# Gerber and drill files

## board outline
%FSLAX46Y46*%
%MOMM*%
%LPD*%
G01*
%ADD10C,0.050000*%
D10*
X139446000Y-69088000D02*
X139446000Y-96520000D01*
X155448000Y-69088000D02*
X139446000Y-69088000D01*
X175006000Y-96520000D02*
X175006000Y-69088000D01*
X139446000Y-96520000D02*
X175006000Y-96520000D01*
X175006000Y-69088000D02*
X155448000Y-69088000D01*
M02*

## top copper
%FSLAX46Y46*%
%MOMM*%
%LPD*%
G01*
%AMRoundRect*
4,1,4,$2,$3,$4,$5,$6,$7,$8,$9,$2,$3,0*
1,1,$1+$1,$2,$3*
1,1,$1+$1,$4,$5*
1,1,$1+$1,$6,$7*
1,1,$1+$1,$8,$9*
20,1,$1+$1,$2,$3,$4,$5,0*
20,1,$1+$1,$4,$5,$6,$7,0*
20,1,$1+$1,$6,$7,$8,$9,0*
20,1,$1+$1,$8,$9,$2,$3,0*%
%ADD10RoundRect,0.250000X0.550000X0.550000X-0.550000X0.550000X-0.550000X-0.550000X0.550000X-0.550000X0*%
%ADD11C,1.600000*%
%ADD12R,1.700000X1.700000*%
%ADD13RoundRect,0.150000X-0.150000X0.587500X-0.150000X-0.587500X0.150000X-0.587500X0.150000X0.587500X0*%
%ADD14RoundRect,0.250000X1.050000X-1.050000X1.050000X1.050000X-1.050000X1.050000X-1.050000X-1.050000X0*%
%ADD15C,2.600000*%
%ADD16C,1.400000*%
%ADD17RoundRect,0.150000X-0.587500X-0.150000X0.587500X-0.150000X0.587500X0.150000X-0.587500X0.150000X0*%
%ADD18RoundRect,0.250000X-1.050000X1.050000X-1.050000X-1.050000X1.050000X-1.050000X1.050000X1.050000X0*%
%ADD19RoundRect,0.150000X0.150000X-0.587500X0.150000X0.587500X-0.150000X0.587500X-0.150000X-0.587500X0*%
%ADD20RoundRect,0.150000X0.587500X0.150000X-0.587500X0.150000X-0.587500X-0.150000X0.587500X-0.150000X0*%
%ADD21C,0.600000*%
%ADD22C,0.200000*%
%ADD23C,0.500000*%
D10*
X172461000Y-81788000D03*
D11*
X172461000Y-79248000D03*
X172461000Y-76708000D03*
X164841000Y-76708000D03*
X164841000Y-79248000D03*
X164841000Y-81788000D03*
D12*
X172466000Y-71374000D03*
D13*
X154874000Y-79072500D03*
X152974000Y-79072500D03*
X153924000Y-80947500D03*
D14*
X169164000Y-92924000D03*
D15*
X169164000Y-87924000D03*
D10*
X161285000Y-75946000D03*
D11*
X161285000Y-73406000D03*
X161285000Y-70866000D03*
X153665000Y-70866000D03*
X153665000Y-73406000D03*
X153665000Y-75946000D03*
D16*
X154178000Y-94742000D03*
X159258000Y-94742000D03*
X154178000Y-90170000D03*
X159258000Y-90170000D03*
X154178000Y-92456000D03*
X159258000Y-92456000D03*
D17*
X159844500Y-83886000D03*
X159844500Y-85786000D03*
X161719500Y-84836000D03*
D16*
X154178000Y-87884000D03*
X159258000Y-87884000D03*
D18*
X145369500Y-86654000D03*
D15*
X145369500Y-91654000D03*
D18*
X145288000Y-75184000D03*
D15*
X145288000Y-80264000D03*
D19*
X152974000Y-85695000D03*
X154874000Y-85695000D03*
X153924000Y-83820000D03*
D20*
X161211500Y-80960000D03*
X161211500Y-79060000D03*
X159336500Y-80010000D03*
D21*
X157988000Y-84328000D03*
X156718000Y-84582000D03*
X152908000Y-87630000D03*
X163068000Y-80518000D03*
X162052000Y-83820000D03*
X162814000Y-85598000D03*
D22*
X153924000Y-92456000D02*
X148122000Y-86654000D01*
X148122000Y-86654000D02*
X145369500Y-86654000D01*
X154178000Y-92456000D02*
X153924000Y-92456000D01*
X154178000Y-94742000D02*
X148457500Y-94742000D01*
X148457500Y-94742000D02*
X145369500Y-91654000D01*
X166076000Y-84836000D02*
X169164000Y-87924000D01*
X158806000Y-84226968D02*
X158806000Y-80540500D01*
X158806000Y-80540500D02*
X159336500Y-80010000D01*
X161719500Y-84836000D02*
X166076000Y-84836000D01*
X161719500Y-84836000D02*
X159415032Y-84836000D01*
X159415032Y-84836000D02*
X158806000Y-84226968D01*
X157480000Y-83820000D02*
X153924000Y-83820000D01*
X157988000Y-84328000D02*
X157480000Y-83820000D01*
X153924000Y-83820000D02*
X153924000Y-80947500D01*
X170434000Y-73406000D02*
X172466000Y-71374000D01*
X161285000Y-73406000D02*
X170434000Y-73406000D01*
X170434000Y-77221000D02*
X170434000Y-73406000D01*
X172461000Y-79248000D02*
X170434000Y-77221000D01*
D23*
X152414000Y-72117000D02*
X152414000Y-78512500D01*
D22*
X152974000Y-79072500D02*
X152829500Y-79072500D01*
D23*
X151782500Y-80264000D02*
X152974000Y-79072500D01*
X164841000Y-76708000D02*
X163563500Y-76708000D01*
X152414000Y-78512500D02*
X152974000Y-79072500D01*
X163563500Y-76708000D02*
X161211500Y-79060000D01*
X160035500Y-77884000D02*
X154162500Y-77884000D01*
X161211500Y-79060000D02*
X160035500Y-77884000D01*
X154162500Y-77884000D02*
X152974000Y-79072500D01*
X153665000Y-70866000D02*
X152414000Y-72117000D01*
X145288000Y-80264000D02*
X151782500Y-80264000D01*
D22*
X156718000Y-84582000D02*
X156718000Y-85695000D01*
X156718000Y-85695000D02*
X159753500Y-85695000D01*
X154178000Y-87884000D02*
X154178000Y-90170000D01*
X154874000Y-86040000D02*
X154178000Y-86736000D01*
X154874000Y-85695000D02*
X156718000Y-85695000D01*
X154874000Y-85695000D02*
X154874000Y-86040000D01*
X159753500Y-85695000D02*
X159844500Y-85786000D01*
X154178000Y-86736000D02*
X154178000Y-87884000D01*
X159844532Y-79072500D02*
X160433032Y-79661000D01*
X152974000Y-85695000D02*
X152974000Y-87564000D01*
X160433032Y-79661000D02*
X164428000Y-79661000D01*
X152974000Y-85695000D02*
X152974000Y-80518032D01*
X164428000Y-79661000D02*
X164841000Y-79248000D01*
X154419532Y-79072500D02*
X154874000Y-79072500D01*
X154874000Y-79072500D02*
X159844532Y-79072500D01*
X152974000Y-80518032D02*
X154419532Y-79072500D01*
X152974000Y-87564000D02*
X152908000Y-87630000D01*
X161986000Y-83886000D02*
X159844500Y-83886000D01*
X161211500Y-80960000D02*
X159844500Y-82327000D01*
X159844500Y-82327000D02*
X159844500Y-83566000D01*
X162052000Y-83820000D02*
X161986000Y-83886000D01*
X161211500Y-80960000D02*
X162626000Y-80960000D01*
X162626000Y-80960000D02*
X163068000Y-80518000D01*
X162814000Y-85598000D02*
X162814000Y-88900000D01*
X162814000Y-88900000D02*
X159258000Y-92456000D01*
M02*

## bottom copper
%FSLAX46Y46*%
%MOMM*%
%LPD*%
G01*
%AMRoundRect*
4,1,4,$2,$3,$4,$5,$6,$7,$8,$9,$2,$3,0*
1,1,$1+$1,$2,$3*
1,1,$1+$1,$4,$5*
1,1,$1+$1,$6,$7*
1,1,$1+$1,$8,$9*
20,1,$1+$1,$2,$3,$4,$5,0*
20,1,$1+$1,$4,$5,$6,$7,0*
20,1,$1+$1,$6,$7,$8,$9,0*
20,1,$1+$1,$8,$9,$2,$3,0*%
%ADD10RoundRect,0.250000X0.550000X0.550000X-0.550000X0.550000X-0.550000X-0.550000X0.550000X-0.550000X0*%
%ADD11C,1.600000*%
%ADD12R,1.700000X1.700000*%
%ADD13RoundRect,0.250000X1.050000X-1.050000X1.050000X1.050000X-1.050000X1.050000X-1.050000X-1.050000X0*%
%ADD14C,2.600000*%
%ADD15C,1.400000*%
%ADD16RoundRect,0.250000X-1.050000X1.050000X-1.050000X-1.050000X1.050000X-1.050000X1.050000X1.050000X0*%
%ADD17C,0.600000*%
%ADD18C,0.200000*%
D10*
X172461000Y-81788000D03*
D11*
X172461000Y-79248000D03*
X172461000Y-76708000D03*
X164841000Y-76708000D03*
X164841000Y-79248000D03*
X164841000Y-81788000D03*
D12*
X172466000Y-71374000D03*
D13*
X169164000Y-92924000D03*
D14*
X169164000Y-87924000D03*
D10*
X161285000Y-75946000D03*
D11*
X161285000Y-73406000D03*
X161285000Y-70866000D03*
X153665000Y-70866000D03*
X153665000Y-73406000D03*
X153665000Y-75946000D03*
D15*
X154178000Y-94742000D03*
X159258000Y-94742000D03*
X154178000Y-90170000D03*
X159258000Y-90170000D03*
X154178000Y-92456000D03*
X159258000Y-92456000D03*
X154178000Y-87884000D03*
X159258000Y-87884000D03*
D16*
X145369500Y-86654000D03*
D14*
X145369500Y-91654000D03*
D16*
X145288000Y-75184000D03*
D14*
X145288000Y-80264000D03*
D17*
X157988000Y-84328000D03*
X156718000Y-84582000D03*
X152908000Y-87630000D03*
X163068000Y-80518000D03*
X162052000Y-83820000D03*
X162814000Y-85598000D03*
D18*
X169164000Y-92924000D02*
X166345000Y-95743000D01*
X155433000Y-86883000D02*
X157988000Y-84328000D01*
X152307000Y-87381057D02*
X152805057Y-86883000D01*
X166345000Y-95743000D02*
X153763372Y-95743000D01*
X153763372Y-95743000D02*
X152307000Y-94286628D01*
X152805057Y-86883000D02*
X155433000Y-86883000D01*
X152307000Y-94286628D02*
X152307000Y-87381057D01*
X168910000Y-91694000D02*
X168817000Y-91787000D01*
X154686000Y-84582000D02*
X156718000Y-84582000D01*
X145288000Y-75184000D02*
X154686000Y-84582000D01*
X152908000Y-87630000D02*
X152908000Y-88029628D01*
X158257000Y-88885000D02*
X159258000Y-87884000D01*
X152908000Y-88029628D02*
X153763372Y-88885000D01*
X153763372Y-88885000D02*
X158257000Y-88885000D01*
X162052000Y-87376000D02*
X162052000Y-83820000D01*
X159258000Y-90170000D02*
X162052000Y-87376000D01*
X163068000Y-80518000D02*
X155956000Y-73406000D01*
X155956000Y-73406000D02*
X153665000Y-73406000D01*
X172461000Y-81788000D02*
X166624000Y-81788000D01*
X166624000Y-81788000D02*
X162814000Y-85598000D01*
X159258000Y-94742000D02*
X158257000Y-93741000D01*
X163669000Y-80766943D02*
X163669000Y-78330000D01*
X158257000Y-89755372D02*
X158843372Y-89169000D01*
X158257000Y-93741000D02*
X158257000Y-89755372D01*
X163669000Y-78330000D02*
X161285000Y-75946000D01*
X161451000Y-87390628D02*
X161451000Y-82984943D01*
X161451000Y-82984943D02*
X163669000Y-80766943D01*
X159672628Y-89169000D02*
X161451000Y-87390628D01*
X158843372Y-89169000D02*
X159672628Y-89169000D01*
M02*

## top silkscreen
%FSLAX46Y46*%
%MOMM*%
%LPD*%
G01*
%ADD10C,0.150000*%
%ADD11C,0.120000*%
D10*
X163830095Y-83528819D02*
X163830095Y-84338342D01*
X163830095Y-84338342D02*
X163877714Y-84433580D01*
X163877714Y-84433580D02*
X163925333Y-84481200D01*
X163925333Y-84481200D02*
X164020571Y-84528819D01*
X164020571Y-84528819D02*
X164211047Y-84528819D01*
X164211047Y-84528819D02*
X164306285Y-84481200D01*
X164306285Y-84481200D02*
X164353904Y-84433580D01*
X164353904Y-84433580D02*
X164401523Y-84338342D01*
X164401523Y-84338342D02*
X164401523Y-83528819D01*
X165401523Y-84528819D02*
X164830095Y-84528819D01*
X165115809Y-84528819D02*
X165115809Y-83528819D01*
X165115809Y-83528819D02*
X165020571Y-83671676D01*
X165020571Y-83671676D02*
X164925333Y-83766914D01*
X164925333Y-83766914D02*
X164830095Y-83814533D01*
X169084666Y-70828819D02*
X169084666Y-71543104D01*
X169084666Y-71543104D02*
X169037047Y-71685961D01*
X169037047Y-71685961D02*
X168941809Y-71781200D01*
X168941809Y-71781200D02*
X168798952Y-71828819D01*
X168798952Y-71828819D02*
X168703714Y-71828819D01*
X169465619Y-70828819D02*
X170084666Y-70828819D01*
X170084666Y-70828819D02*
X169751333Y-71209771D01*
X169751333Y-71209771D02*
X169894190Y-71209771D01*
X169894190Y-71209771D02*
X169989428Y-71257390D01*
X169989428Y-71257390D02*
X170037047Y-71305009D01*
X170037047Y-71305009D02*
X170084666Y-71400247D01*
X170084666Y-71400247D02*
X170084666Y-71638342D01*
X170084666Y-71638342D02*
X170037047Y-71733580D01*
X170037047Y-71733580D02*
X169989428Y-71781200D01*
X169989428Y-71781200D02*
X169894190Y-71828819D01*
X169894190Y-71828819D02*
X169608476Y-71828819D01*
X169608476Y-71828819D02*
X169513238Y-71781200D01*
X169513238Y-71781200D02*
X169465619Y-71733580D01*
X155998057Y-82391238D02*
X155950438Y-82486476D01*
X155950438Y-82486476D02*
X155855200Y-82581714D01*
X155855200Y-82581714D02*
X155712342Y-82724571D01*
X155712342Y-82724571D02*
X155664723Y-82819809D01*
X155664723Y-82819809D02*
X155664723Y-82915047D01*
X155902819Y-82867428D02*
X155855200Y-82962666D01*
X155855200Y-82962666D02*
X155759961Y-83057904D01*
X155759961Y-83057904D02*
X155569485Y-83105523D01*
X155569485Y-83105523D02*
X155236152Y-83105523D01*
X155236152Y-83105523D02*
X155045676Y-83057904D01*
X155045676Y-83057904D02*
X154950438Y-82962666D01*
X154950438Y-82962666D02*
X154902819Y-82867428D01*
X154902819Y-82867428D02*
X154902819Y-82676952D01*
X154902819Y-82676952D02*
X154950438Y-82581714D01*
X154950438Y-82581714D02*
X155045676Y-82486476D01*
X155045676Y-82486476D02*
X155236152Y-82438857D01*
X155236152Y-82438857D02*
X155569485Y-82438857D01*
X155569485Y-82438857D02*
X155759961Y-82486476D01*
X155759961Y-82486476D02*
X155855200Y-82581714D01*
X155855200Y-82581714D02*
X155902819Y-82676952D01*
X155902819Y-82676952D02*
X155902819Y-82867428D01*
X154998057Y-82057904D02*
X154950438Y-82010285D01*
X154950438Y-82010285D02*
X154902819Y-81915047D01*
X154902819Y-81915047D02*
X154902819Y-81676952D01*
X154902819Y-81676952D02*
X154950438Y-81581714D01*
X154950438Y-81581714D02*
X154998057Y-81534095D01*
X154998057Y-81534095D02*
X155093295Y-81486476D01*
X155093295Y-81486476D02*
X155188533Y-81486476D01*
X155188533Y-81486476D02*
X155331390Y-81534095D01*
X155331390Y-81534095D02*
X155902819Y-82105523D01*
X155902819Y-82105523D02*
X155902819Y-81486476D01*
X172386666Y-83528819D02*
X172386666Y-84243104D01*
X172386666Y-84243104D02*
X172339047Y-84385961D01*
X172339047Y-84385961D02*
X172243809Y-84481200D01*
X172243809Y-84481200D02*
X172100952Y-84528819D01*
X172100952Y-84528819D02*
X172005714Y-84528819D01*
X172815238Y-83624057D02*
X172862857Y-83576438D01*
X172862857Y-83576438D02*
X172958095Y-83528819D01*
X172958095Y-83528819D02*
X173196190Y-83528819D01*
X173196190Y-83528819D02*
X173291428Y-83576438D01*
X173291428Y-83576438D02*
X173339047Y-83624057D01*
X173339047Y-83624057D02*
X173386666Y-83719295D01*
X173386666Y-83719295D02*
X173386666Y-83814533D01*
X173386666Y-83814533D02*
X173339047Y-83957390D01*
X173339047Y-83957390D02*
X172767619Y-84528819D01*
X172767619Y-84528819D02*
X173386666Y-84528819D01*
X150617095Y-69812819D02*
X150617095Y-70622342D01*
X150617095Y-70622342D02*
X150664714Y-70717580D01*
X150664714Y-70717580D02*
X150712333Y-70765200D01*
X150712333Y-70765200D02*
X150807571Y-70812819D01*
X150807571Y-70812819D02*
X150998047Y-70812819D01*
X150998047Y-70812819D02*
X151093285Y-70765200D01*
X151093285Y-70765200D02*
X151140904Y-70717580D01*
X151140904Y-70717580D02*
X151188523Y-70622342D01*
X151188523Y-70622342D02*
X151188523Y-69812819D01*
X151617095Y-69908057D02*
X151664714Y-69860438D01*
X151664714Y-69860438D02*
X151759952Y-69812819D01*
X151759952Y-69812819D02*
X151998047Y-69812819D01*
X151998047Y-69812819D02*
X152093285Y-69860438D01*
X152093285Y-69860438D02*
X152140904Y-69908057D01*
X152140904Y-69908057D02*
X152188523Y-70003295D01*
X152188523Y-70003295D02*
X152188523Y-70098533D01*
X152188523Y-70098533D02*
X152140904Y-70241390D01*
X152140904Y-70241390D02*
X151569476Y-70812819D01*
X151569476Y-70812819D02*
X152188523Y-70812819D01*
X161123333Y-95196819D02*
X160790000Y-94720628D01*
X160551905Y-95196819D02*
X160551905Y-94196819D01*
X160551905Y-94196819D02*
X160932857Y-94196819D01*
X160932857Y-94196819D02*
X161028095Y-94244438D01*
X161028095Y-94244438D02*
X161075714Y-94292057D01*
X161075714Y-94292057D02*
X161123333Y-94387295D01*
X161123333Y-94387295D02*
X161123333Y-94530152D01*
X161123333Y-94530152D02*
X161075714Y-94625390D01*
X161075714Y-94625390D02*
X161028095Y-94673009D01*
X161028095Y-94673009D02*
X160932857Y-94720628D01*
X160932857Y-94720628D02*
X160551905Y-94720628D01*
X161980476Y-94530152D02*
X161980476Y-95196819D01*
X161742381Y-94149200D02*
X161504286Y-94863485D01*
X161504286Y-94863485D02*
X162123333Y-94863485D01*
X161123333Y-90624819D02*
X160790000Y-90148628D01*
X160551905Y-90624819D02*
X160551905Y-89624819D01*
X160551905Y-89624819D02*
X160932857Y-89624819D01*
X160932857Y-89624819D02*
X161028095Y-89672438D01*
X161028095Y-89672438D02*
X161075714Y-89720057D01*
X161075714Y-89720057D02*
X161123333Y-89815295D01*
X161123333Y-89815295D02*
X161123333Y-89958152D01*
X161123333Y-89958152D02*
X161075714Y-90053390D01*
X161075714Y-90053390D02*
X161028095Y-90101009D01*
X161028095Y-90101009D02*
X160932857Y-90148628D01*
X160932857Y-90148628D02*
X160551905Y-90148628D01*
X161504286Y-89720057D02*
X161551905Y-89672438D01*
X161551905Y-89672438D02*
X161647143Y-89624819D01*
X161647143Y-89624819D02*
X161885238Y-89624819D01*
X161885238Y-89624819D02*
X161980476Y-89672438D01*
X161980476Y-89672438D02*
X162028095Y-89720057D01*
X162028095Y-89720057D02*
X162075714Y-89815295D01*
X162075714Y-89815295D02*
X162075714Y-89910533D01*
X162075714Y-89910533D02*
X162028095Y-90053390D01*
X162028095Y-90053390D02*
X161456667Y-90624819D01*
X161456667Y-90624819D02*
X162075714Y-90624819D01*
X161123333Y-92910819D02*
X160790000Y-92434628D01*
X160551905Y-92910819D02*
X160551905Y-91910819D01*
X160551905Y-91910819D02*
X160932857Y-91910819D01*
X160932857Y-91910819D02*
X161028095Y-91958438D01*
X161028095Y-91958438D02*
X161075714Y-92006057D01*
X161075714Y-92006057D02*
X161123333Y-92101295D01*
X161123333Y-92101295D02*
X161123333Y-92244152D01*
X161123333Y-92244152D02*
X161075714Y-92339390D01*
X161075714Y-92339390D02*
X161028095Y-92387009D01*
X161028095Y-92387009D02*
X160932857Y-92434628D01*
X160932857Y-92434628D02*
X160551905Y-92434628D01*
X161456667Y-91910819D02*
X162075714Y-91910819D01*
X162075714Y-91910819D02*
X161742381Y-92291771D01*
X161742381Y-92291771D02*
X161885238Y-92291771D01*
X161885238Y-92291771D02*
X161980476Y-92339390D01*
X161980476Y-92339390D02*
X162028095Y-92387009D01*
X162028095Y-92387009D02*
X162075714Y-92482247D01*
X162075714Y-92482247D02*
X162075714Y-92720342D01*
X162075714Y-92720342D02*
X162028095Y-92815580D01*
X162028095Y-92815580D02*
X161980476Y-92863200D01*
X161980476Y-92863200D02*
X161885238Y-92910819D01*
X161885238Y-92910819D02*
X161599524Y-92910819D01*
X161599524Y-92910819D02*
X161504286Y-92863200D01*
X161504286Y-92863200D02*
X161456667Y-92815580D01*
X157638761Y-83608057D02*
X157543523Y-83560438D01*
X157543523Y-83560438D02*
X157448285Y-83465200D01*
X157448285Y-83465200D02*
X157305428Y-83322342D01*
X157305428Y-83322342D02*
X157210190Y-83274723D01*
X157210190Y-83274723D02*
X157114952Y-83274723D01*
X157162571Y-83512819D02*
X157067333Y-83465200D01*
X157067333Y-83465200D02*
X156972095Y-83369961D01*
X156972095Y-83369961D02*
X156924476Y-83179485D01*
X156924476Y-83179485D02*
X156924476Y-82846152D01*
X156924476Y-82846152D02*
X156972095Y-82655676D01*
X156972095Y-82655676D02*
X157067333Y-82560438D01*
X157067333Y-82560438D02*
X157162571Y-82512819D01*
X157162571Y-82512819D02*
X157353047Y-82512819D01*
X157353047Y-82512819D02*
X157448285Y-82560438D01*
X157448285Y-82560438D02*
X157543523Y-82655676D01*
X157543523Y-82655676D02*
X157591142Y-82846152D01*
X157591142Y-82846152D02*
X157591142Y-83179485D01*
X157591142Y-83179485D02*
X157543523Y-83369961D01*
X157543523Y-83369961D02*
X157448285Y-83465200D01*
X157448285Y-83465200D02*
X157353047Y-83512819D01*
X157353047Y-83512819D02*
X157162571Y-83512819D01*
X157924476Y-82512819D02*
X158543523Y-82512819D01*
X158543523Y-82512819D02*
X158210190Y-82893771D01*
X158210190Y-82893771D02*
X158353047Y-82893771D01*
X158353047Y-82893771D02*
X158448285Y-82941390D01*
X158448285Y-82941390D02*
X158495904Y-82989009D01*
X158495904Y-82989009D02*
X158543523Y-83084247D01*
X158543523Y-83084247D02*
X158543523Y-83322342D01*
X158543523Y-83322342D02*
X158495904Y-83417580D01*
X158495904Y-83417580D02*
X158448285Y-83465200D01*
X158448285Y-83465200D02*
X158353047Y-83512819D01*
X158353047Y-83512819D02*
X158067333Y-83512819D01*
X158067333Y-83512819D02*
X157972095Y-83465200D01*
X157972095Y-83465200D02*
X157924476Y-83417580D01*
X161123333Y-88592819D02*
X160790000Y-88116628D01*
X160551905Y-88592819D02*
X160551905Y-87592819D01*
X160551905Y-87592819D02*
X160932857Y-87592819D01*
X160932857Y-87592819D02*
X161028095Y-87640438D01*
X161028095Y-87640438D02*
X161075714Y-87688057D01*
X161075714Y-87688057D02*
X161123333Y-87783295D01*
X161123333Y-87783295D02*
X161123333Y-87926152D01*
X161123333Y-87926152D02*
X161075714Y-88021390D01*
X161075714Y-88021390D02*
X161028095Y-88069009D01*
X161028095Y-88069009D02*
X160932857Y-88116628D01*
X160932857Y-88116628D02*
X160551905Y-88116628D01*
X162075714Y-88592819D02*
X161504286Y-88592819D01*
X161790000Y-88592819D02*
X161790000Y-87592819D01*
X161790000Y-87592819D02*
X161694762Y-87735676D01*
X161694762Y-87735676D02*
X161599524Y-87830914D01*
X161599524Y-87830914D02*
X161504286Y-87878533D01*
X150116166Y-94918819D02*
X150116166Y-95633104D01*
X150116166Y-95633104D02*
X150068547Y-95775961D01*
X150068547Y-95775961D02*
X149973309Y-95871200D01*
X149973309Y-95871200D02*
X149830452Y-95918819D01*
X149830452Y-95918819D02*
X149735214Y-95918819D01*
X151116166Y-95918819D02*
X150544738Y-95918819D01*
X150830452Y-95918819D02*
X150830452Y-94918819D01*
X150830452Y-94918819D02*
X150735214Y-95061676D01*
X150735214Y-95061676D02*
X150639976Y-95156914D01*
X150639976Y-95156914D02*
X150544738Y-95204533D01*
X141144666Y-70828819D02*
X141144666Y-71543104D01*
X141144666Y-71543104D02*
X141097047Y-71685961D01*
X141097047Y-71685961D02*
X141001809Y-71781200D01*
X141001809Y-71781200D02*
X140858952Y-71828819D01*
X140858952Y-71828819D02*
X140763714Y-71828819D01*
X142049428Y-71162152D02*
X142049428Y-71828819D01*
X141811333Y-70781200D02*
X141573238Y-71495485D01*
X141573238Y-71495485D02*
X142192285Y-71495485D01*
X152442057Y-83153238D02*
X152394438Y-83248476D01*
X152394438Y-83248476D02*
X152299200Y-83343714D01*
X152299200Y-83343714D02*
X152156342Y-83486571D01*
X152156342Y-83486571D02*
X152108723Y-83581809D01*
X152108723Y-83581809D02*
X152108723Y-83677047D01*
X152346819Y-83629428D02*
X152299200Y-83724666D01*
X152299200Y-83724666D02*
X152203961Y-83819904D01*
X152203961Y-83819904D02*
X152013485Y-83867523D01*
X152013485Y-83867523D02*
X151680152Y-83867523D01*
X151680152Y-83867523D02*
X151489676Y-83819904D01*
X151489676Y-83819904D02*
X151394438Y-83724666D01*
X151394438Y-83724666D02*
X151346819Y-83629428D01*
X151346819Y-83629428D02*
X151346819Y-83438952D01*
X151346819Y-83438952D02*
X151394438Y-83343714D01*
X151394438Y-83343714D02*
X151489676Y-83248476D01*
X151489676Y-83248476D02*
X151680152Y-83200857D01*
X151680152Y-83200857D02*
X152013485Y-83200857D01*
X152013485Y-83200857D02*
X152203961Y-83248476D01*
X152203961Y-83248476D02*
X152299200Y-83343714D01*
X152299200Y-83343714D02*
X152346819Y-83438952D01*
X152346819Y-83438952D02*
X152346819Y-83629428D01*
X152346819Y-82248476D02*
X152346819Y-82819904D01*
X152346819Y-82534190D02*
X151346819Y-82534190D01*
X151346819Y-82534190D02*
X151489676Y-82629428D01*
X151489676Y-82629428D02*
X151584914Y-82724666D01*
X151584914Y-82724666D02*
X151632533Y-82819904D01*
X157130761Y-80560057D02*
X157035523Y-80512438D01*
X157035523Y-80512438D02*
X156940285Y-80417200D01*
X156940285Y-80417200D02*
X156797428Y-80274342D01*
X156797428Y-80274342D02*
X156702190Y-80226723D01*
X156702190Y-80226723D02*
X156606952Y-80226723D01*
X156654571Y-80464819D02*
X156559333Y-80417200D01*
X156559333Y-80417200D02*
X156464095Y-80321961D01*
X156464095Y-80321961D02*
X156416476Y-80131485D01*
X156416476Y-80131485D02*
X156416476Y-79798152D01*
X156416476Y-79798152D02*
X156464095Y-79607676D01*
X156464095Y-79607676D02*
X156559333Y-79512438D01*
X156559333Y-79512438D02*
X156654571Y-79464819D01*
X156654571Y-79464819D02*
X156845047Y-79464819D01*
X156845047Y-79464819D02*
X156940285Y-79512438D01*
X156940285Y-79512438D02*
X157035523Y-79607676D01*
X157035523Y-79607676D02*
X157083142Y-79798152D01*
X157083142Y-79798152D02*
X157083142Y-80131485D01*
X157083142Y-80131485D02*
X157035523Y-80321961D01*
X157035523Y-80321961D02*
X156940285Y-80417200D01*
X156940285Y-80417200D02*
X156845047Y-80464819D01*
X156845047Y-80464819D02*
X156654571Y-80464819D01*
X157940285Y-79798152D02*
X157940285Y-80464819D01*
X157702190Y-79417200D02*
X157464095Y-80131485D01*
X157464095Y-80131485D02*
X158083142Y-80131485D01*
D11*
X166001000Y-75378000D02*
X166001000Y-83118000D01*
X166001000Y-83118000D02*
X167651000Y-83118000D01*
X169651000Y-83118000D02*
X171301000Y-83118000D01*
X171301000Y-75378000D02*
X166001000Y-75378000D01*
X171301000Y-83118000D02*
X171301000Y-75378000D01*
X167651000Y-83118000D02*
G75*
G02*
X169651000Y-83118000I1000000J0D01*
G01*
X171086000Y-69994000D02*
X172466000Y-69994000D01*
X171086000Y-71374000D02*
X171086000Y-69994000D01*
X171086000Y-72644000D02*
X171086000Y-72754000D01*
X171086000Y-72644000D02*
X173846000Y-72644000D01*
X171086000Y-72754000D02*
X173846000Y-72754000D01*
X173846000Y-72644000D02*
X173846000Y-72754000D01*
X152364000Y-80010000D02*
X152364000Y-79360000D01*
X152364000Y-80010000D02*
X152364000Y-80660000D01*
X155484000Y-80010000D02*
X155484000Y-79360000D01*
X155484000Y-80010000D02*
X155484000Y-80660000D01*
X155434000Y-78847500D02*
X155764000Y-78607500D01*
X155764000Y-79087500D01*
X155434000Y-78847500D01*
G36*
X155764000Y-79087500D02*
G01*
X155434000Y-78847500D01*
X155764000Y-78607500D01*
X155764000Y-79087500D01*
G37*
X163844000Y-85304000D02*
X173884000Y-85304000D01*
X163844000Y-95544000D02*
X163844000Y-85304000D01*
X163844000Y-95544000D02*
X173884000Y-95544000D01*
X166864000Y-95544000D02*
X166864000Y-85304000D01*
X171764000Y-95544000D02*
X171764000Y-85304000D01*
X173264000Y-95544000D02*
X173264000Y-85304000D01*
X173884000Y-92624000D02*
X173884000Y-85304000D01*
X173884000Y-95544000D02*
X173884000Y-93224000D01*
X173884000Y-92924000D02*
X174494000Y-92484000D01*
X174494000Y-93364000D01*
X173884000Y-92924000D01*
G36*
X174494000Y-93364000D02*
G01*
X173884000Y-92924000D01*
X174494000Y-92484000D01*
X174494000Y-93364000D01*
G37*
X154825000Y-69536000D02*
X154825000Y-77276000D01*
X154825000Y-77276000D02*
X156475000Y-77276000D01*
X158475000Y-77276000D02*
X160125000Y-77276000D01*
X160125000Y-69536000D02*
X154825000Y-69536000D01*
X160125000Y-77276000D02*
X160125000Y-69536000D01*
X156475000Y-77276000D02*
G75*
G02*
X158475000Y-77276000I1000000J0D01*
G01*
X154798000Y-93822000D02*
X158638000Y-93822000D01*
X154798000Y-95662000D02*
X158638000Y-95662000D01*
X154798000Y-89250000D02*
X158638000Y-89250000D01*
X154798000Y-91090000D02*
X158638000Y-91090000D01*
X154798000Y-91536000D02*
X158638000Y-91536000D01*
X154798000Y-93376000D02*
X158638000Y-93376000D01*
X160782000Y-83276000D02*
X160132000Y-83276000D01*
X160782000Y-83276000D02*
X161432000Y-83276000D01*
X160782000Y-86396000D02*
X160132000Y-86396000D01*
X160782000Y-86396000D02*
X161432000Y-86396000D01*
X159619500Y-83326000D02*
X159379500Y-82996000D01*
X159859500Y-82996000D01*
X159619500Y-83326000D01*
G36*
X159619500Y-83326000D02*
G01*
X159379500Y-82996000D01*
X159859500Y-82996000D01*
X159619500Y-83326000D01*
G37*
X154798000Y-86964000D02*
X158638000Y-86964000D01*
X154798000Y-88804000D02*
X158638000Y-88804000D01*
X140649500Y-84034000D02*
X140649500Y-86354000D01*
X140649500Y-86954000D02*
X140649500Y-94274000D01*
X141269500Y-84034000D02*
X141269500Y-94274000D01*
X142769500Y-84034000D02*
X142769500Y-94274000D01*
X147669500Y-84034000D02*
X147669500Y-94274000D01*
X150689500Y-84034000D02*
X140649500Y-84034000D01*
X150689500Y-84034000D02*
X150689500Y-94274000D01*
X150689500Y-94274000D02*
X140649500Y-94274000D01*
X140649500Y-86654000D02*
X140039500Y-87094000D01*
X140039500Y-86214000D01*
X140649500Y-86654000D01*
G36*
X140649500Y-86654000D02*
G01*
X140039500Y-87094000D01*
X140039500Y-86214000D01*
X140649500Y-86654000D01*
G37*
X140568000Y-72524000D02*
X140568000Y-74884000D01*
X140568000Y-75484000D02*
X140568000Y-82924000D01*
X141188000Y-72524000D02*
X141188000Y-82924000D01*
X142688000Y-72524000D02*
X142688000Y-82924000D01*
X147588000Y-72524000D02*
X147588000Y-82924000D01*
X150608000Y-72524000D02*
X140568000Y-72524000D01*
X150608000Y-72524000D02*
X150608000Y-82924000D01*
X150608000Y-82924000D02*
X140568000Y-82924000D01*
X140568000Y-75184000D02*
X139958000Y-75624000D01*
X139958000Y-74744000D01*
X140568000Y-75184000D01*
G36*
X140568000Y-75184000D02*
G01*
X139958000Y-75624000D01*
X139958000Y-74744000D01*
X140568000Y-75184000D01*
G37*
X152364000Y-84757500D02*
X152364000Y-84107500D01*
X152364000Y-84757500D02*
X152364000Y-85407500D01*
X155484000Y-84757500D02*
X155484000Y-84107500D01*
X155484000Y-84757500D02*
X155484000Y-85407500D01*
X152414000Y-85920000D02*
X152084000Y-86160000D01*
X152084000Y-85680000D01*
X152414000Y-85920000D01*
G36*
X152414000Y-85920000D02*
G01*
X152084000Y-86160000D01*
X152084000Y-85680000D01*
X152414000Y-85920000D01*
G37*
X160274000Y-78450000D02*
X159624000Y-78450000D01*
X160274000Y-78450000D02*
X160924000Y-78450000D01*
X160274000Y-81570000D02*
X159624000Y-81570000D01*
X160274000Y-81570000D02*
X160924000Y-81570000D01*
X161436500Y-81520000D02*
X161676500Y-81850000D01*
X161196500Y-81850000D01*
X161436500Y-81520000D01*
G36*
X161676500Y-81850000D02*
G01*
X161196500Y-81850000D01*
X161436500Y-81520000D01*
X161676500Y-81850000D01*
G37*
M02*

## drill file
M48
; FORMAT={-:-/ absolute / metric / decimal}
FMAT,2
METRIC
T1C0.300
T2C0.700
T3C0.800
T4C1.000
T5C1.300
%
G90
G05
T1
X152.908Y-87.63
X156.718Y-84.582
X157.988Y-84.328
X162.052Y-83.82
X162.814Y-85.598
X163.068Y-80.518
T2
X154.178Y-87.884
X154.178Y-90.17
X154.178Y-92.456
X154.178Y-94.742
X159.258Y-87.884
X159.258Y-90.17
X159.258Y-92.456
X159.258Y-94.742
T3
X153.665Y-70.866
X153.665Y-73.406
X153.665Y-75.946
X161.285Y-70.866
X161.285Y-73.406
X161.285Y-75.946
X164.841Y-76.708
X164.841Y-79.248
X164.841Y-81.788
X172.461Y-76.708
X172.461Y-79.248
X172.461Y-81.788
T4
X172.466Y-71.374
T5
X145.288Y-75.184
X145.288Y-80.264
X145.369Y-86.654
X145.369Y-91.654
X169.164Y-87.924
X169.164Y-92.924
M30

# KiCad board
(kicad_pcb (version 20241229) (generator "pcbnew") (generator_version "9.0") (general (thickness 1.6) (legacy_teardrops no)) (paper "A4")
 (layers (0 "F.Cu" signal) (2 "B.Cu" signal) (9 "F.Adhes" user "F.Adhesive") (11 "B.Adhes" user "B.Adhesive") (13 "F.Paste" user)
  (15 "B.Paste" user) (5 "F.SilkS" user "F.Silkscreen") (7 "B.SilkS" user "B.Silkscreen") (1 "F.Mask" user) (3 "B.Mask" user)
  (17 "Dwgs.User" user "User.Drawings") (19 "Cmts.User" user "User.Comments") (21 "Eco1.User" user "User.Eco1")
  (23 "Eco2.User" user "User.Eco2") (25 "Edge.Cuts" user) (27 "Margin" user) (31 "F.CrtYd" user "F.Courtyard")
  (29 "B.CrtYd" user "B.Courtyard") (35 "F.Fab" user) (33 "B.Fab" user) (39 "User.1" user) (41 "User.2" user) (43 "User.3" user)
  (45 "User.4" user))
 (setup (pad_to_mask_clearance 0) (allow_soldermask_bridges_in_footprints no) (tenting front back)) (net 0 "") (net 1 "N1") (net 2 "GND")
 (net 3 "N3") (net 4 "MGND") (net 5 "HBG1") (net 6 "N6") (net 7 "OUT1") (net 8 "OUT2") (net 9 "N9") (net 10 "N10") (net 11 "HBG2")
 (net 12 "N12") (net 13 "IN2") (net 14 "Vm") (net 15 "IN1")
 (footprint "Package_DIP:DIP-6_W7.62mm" (layer "F.Cu") (at 172.461 81.788 180)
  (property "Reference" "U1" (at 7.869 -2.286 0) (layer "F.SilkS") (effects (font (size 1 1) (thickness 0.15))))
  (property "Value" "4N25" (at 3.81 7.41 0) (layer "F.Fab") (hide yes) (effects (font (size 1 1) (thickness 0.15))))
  (fp_line (start 6.46 6.41) (end 6.46 -1.33) (stroke (width 0.12) (type solid)) (layer "F.SilkS"))
  (fp_line (start 6.46 -1.33) (end 4.81 -1.33) (stroke (width 0.12) (type solid)) (layer "F.SilkS"))
  (fp_line (start 2.81 -1.33) (end 1.16 -1.33) (stroke (width 0.12) (type solid)) (layer "F.SilkS"))
  (fp_line (start 1.16 6.41) (end 6.46 6.41) (stroke (width 0.12) (type solid)) (layer "F.SilkS"))
  (fp_line (start 1.16 -1.33) (end 1.16 6.41) (stroke (width 0.12) (type solid)) (layer "F.SilkS"))
  (fp_arc (start 4.81 -1.33) (mid 3.81 -0.33) (end 2.81 -1.33) (stroke (width 0.12) (type solid)) (layer "F.SilkS"))
  (pad "1" thru_hole roundrect (at 0 0 180) (size 1.6 1.6) (drill 0.8) (layers "*.Cu" "*.Mask") (remove_unused_layers no)
   (roundrect_rratio 0.15625) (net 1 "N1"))
  (pad "2" thru_hole circle (at 0 2.54 180) (size 1.6 1.6) (drill 0.8) (layers "*.Cu" "*.Mask") (remove_unused_layers no) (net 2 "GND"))
  (pad "3" thru_hole circle (at 0 5.08 180) (size 1.6 1.6) (drill 0.8) (layers "*.Cu" "*.Mask") (remove_unused_layers no) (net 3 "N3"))
  (pad "4" thru_hole circle (at 7.62 5.08 180) (size 1.6 1.6) (drill 0.8) (layers "*.Cu" "*.Mask") (remove_unused_layers no) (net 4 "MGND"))
  (pad "5" thru_hole circle (at 7.62 2.54 180) (size 1.6 1.6) (drill 0.8) (layers "*.Cu" "*.Mask") (remove_unused_layers no) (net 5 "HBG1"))
  (pad "6" thru_hole circle (at 7.62 0 180) (size 1.6 1.6) (drill 0.8) (layers "*.Cu" "*.Mask") (remove_unused_layers no) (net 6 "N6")))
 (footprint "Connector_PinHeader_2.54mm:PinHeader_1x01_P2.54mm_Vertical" (layer "F.Cu") (at 172.466 71.374)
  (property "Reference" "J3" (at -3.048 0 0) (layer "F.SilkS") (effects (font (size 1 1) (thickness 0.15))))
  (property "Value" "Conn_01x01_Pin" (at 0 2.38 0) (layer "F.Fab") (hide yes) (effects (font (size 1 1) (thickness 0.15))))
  (fp_line (start -1.38 -1.38) (end 0 -1.38) (stroke (width 0.12) (type solid)) (layer "F.SilkS"))
  (fp_line (start -1.38 0) (end -1.38 -1.38) (stroke (width 0.12) (type solid)) (layer "F.SilkS"))
  (fp_line (start -1.38 1.27) (end -1.38 1.38) (stroke (width 0.12) (type solid)) (layer "F.SilkS"))
  (fp_line (start -1.38 1.27) (end 1.38 1.27) (stroke (width 0.12) (type solid)) (layer "F.SilkS"))
  (fp_line (start -1.38 1.38) (end 1.38 1.38) (stroke (width 0.12) (type solid)) (layer "F.SilkS"))
  (fp_line (start 1.38 1.27) (end 1.38 1.38) (stroke (width 0.12) (type solid)) (layer "F.SilkS"))
  (pad "1" thru_hole rect (at 0 0) (size 1.7 1.7) (drill 1) (layers "*.Cu" "*.Mask") (remove_unused_layers no) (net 2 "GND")))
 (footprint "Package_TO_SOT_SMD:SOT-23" (layer "F.Cu") (at 153.924 80.01 -90)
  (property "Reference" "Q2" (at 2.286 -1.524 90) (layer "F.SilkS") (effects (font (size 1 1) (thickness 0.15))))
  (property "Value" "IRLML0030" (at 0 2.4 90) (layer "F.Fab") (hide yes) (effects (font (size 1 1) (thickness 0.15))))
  (fp_line (start 0 1.56) (end -0.65 1.56) (stroke (width 0.12) (type solid)) (layer "F.SilkS"))
  (fp_line (start 0 1.56) (end 0.65 1.56) (stroke (width 0.12) (type solid)) (layer "F.SilkS"))
  (fp_line (start 0 -1.56) (end -0.65 -1.56) (stroke (width 0.12) (type solid)) (layer "F.SilkS"))
  (fp_line (start 0 -1.56) (end 0.65 -1.56) (stroke (width 0.12) (type solid)) (layer "F.SilkS"))
  (fp_poly (pts (xy -1.1625 -1.51) (xy -1.4025 -1.84) (xy -0.9225 -1.84)) (stroke (width 0.12) (type solid)) (fill yes) (layer "F.SilkS"))
  (pad "1" smd roundrect (at -0.9375 -0.95 270) (size 1.475 0.6) (layers "F.Cu" "F.Mask" "F.Paste") (roundrect_rratio 0.25) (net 5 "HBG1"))
  (pad "2" smd roundrect (at -0.9375 0.95 270) (size 1.475 0.6) (layers "F.Cu" "F.Mask" "F.Paste") (roundrect_rratio 0.25) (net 4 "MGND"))
  (pad "3" smd roundrect (at 0.9375 0 270) (size 1.475 0.6) (layers "F.Cu" "F.Mask" "F.Paste") (roundrect_rratio 0.25) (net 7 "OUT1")))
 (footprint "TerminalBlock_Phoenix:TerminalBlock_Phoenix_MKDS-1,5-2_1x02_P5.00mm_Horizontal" (layer "F.Cu") (at 169.164 92.924 90)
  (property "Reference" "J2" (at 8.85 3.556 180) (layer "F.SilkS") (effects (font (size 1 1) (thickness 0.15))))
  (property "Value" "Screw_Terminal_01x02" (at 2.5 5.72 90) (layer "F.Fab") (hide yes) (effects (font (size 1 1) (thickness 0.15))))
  (fp_line (start 7.62 -5.32) (end 7.62 4.72) (stroke (width 0.12) (type solid)) (layer "F.SilkS"))
  (fp_line (start -2.62 -5.32) (end 7.62 -5.32) (stroke (width 0.12) (type solid)) (layer "F.SilkS"))
  (fp_line (start -2.62 -5.32) (end -2.62 4.72) (stroke (width 0.12) (type solid)) (layer "F.SilkS"))
  (fp_line (start -2.62 -2.3) (end 7.62 -2.3) (stroke (width 0.12) (type solid)) (layer "F.SilkS"))
  (fp_line (start -2.62 2.6) (end 7.62 2.6) (stroke (width 0.12) (type solid)) (layer "F.SilkS"))
  (fp_line (start -2.62 4.1) (end 7.62 4.1) (stroke (width 0.12) (type solid)) (layer "F.SilkS"))
  (fp_line (start 0.3 4.72) (end 7.62 4.72) (stroke (width 0.12) (type solid)) (layer "F.SilkS"))
  (fp_line (start -2.62 4.72) (end -0.3 4.72) (stroke (width 0.12) (type solid)) (layer "F.SilkS"))
  (fp_poly (pts (xy 0 4.72) (xy 0.44 5.33) (xy -0.44 5.33)) (stroke (width 0.12) (type solid)) (fill yes) (layer "F.SilkS"))
  (pad "1" thru_hole roundrect (at 0 0 90) (size 2.6 2.6) (drill 1.3) (layers "*.Cu" "*.Mask") (remove_unused_layers no)
   (roundrect_rratio 0.096154) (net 7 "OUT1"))
  (pad "2" thru_hole circle (at 5 0 90) (size 2.6 2.6) (drill 1.3) (layers "*.Cu" "*.Mask") (remove_unused_layers no) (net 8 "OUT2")))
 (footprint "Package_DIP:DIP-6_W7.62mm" (layer "F.Cu") (at 161.285 75.946 180)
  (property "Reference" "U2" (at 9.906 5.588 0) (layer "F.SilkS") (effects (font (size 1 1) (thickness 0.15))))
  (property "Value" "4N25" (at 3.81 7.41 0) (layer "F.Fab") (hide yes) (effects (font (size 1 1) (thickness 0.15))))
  (fp_line (start 6.46 6.41) (end 6.46 -1.33) (stroke (width 0.12) (type solid)) (layer "F.SilkS"))
  (fp_line (start 6.46 -1.33) (end 4.81 -1.33) (stroke (width 0.12) (type solid)) (layer "F.SilkS"))
  (fp_line (start 2.81 -1.33) (end 1.16 -1.33) (stroke (width 0.12) (type solid)) (layer "F.SilkS"))
  (fp_line (start 1.16 6.41) (end 6.46 6.41) (stroke (width 0.12) (type solid)) (layer "F.SilkS"))
  (fp_line (start 1.16 -1.33) (end 1.16 6.41) (stroke (width 0.12) (type solid)) (layer "F.SilkS"))
  (fp_arc (start 4.81 -1.33) (mid 3.81 -0.33) (end 2.81 -1.33) (stroke (width 0.12) (type solid)) (layer "F.SilkS"))
  (pad "1" thru_hole roundrect (at 0 0 180) (size 1.6 1.6) (drill 0.8) (layers "*.Cu" "*.Mask") (remove_unused_layers no)
   (roundrect_rratio 0.15625) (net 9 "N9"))
  (pad "2" thru_hole circle (at 0 2.54 180) (size 1.6 1.6) (drill 0.8) (layers "*.Cu" "*.Mask") (remove_unused_layers no) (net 2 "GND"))
  (pad "3" thru_hole circle (at 0 5.08 180) (size 1.6 1.6) (drill 0.8) (layers "*.Cu" "*.Mask") (remove_unused_layers no) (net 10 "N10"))
  (pad "4" thru_hole circle (at 7.62 5.08 180) (size 1.6 1.6) (drill 0.8) (layers "*.Cu" "*.Mask") (remove_unused_layers no) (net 4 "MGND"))
  (pad "5" thru_hole circle (at 7.62 2.54 180) (size 1.6 1.6) (drill 0.8) (layers "*.Cu" "*.Mask") (remove_unused_layers no) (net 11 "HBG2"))
  (pad "6" thru_hole circle (at 7.62 0 180) (size 1.6 1.6) (drill 0.8) (layers "*.Cu" "*.Mask") (remove_unused_layers no) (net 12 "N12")))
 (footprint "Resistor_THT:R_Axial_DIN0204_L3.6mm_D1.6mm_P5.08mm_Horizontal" (layer "F.Cu") (at 154.178 94.742)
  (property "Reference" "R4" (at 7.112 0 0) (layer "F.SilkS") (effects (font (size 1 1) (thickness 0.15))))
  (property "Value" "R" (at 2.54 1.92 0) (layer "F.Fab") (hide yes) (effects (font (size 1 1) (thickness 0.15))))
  (fp_line (start 0.62 -0.92) (end 4.46 -0.92) (stroke (width 0.12) (type solid)) (layer "F.SilkS"))
  (fp_line (start 0.62 0.92) (end 4.46 0.92) (stroke (width 0.12) (type solid)) (layer "F.SilkS"))
  (pad "1" thru_hole circle (at 0 0) (size 1.4 1.4) (drill 0.7) (layers "*.Cu" "*.Mask") (remove_unused_layers no) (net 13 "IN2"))
  (pad "2" thru_hole circle (at 5.08 0) (size 1.4 1.4) (drill 0.7) (layers "*.Cu" "*.Mask") (remove_unused_layers no) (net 9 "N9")))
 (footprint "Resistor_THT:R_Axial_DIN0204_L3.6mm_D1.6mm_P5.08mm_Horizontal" (layer "F.Cu") (at 154.178 90.17)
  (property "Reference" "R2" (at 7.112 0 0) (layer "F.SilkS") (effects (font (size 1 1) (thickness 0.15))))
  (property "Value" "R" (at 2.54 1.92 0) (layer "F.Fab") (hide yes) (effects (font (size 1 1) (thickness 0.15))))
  (fp_line (start 0.62 -0.92) (end 4.46 -0.92) (stroke (width 0.12) (type solid)) (layer "F.SilkS"))
  (fp_line (start 0.62 0.92) (end 4.46 0.92) (stroke (width 0.12) (type solid)) (layer "F.SilkS"))
  (pad "1" thru_hole circle (at 0 0) (size 1.4 1.4) (drill 0.7) (layers "*.Cu" "*.Mask") (remove_unused_layers no) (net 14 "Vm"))
  (pad "2" thru_hole circle (at 5.08 0) (size 1.4 1.4) (drill 0.7) (layers "*.Cu" "*.Mask") (remove_unused_layers no) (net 11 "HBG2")))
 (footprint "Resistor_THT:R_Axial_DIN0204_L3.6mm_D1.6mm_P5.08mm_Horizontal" (layer "F.Cu") (at 154.178 92.456)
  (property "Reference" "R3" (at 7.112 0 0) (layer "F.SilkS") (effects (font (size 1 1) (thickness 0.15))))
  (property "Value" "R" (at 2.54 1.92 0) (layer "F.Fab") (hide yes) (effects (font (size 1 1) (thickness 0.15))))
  (fp_line (start 0.62 -0.92) (end 4.46 -0.92) (stroke (width 0.12) (type solid)) (layer "F.SilkS"))
  (fp_line (start 0.62 0.92) (end 4.46 0.92) (stroke (width 0.12) (type solid)) (layer "F.SilkS"))
  (pad "1" thru_hole circle (at 0 0) (size 1.4 1.4) (drill 0.7) (layers "*.Cu" "*.Mask") (remove_unused_layers no) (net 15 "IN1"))
  (pad "2" thru_hole circle (at 5.08 0) (size 1.4 1.4) (drill 0.7) (layers "*.Cu" "*.Mask") (remove_unused_layers no) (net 1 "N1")))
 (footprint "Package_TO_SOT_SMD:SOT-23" (layer "F.Cu") (at 160.782 84.836)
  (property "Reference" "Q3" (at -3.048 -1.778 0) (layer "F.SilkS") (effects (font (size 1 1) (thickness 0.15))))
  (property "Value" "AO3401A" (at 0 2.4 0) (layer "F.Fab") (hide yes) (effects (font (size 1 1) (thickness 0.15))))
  (fp_line (start 0 -1.56) (end -0.65 -1.56) (stroke (width 0.12) (type solid)) (layer "F.SilkS"))
  (fp_line (start 0 -1.56) (end 0.65 -1.56) (stroke (width 0.12) (type solid)) (layer "F.SilkS"))
  (fp_line (start 0 1.56) (end -0.65 1.56) (stroke (width 0.12) (type solid)) (layer "F.SilkS"))
  (fp_line (start 0 1.56) (end 0.65 1.56) (stroke (width 0.12) (type solid)) (layer "F.SilkS"))
  (fp_poly (pts (xy -1.1625 -1.51) (xy -1.4025 -1.84) (xy -0.9225 -1.84)) (stroke (width 0.12) (type solid)) (fill yes) (layer "F.SilkS"))
  (pad "1" smd roundrect (at -0.9375 -0.95) (size 1.475 0.6) (layers "F.Cu" "F.Mask" "F.Paste") (roundrect_rratio 0.25) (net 11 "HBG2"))
  (pad "2" smd roundrect (at -0.9375 0.95) (size 1.475 0.6) (layers "F.Cu" "F.Mask" "F.Paste") (roundrect_rratio 0.25) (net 14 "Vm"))
  (pad "3" smd roundrect (at 0.9375 0) (size 1.475 0.6) (layers "F.Cu" "F.Mask" "F.Paste") (roundrect_rratio 0.25) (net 8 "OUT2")))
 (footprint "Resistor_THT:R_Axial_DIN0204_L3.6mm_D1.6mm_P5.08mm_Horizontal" (layer "F.Cu") (at 154.178 87.884)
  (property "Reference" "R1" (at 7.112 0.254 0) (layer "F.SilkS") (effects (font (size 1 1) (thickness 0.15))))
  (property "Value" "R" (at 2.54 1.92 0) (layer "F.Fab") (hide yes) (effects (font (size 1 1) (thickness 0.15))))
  (fp_line (start 0.62 -0.92) (end 4.46 -0.92) (stroke (width 0.12) (type solid)) (layer "F.SilkS"))
  (fp_line (start 0.62 0.92) (end 4.46 0.92) (stroke (width 0.12) (type solid)) (layer "F.SilkS"))
  (pad "1" thru_hole circle (at 0 0) (size 1.4 1.4) (drill 0.7) (layers "*.Cu" "*.Mask") (remove_unused_layers no) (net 14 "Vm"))
  (pad "2" thru_hole circle (at 5.08 0) (size 1.4 1.4) (drill 0.7) (layers "*.Cu" "*.Mask") (remove_unused_layers no) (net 5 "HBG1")))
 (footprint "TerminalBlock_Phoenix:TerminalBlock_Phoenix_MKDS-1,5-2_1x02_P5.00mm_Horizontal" (layer "F.Cu") (at 145.3695 86.654 -90)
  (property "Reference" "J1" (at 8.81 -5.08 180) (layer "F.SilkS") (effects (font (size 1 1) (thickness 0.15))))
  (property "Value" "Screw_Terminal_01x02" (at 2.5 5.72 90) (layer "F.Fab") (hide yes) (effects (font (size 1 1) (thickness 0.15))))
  (fp_line (start -2.62 4.72) (end -0.3 4.72) (stroke (width 0.12) (type solid)) (layer "F.SilkS"))
  (fp_line (start 0.3 4.72) (end 7.62 4.72) (stroke (width 0.12) (type solid)) (layer "F.SilkS"))
  (fp_line (start -2.62 4.1) (end 7.62 4.1) (stroke (width 0.12) (type solid)) (layer "F.SilkS"))
  (fp_line (start -2.62 2.6) (end 7.62 2.6) (stroke (width 0.12) (type solid)) (layer "F.SilkS"))
  (fp_line (start -2.62 -2.3) (end 7.62 -2.3) (stroke (width 0.12) (type solid)) (layer "F.SilkS"))
  (fp_line (start -2.62 -5.32) (end -2.62 4.72) (stroke (width 0.12) (type solid)) (layer "F.SilkS"))
  (fp_line (start -2.62 -5.32) (end 7.62 -5.32) (stroke (width 0.12) (type solid)) (layer "F.SilkS"))
  (fp_line (start 7.62 -5.32) (end 7.62 4.72) (stroke (width 0.12) (type solid)) (layer "F.SilkS"))
  (fp_poly (pts (xy 0 4.72) (xy 0.44 5.33) (xy -0.44 5.33)) (stroke (width 0.12) (type solid)) (fill yes) (layer "F.SilkS"))
  (pad "1" thru_hole roundrect (at 0 0 270) (size 2.6 2.6) (drill 1.3) (layers "*.Cu" "*.Mask") (remove_unused_layers no)
   (roundrect_rratio 0.096154) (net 15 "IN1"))
  (pad "2" thru_hole circle (at 5 0 270) (size 2.6 2.6) (drill 1.3) (layers "*.Cu" "*.Mask") (remove_unused_layers no) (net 13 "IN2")))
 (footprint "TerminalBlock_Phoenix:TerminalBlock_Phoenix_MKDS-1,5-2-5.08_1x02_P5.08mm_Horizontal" (layer "F.Cu") (at 145.288 75.184 -90)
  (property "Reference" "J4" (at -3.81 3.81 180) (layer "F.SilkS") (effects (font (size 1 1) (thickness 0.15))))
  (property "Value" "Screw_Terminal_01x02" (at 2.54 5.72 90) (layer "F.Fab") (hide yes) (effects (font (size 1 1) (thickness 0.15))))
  (fp_line (start -2.66 4.72) (end -0.3 4.72) (stroke (width 0.12) (type solid)) (layer "F.SilkS"))
  (fp_line (start 0.3 4.72) (end 7.74 4.72) (stroke (width 0.12) (type solid)) (layer "F.SilkS"))
  (fp_line (start -2.66 4.1) (end 7.74 4.1) (stroke (width 0.12) (type solid)) (layer "F.SilkS"))
  (fp_line (start -2.66 2.6) (end 7.74 2.6) (stroke (width 0.12) (type solid)) (layer "F.SilkS"))
  (fp_line (start -2.66 -2.3) (end 7.74 -2.3) (stroke (width 0.12) (type solid)) (layer "F.SilkS"))
  (fp_line (start -2.66 -5.32) (end -2.66 4.72) (stroke (width 0.12) (type solid)) (layer "F.SilkS"))
  (fp_line (start -2.66 -5.32) (end 7.74 -5.32) (stroke (width 0.12) (type solid)) (layer "F.SilkS"))
  (fp_line (start 7.74 -5.32) (end 7.74 4.72) (stroke (width 0.12) (type solid)) (layer "F.SilkS"))
  (fp_poly (pts (xy 0 4.72) (xy 0.44 5.33) (xy -0.44 5.33)) (stroke (width 0.12) (type solid)) (fill yes) (layer "F.SilkS"))
  (pad "1" thru_hole roundrect (at 0 0 270) (size 2.6 2.6) (drill 1.3) (layers "*.Cu" "*.Mask") (remove_unused_layers no)
   (roundrect_rratio 0.096154) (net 14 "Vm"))
  (pad "2" thru_hole circle (at 5.08 0 270) (size 2.6 2.6) (drill 1.3) (layers "*.Cu" "*.Mask") (remove_unused_layers no) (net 4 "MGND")))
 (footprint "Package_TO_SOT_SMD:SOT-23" (layer "F.Cu") (at 153.924 84.7575 90)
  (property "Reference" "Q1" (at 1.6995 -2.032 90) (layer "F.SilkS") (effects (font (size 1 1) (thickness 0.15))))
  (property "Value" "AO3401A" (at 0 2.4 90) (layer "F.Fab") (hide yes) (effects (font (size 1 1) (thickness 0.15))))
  (fp_line (start 0 -1.56) (end 0.65 -1.56) (stroke (width 0.12) (type solid)) (layer "F.SilkS"))
  (fp_line (start 0 -1.56) (end -0.65 -1.56) (stroke (width 0.12) (type solid)) (layer "F.SilkS"))
  (fp_line (start 0 1.56) (end 0.65 1.56) (stroke (width 0.12) (type solid)) (layer "F.SilkS"))
  (fp_line (start 0 1.56) (end -0.65 1.56) (stroke (width 0.12) (type solid)) (layer "F.SilkS"))
  (fp_poly (pts (xy -1.1625 -1.51) (xy -1.4025 -1.84) (xy -0.9225 -1.84)) (stroke (width 0.12) (type solid)) (fill yes) (layer "F.SilkS"))
  (pad "1" smd roundrect (at -0.9375 -0.95 90) (size 1.475 0.6) (layers "F.Cu" "F.Mask" "F.Paste") (roundrect_rratio 0.25) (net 5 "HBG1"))
  (pad "2" smd roundrect (at -0.9375 0.95 90) (size 1.475 0.6) (layers "F.Cu" "F.Mask" "F.Paste") (roundrect_rratio 0.25) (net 14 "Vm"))
  (pad "3" smd roundrect (at 0.9375 0 90) (size 1.475 0.6) (layers "F.Cu" "F.Mask" "F.Paste") (roundrect_rratio 0.25) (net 7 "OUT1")))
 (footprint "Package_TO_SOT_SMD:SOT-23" (layer "F.Cu") (at 160.274 80.01 180)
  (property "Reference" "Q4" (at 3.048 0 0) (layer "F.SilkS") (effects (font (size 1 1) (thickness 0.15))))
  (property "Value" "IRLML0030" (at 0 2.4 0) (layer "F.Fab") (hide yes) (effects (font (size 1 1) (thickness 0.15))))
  (fp_line (start 0 1.56) (end 0.65 1.56) (stroke (width 0.12) (type solid)) (layer "F.SilkS"))
  (fp_line (start 0 1.56) (end -0.65 1.56) (stroke (width 0.12) (type solid)) (layer "F.SilkS"))
  (fp_line (start 0 -1.56) (end 0.65 -1.56) (stroke (width 0.12) (type solid)) (layer "F.SilkS"))
  (fp_line (start 0 -1.56) (end -0.65 -1.56) (stroke (width 0.12) (type solid)) (layer "F.SilkS"))
  (fp_poly (pts (xy -1.1625 -1.51) (xy -1.4025 -1.84) (xy -0.9225 -1.84)) (stroke (width 0.12) (type solid)) (fill yes) (layer "F.SilkS"))
  (pad "1" smd roundrect (at -0.9375 -0.95 180) (size 1.475 0.6) (layers "F.Cu" "F.Mask" "F.Paste") (roundrect_rratio 0.25) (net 11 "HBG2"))
  (pad "2" smd roundrect (at -0.9375 0.95 180) (size 1.475 0.6) (layers "F.Cu" "F.Mask" "F.Paste") (roundrect_rratio 0.25) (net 4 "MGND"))
  (pad "3" smd roundrect (at 0.9375 0 180) (size 1.475 0.6) (layers "F.Cu" "F.Mask" "F.Paste") (roundrect_rratio 0.25) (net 8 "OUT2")))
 (gr_line (start 139.446 69.088) (end 139.446 96.52) (stroke (width 0.05) (type default)) (layer "Edge.Cuts"))
 (gr_line (start 155.448 69.088) (end 139.446 69.088) (stroke (width 0.05) (type default)) (layer "Edge.Cuts"))
 (gr_line (start 175.006 96.52) (end 175.006 69.088) (stroke (width 0.05) (type default)) (layer "Edge.Cuts"))
 (gr_line (start 139.446 96.52) (end 175.006 96.52) (stroke (width 0.05) (type default)) (layer "Edge.Cuts"))
 (gr_line (start 175.006 69.088) (end 155.448 69.088) (stroke (width 0.05) (type default)) (layer "Edge.Cuts"))
 (segment (start 153.924 92.456) (end 148.122 86.654) (width 0.2) (layer "F.Cu") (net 15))
 (segment (start 148.122 86.654) (end 145.3695 86.654) (width 0.2) (layer "F.Cu") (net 15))
 (segment (start 154.178 92.456) (end 153.924 92.456) (width 0.2) (layer "F.Cu") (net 15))
 (segment (start 154.178 94.742) (end 148.4575 94.742) (width 0.2) (layer "F.Cu") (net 13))
 (segment (start 148.4575 94.742) (end 145.3695 91.654) (width 0.2) (layer "F.Cu") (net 13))
 (segment (start 166.076 84.836) (end 169.164 87.924) (width 0.2) (layer "F.Cu") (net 8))
 (segment (start 158.806 84.226968) (end 158.806 80.5405) (width 0.2) (layer "F.Cu") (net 8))
 (segment (start 158.806 80.5405) (end 159.3365 80.01) (width 0.2) (layer "F.Cu") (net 8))
 (segment (start 161.7195 84.836) (end 166.076 84.836) (width 0.2) (layer "F.Cu") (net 8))
 (segment (start 161.7195 84.836) (end 159.415032 84.836) (width 0.2) (layer "F.Cu") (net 8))
 (segment (start 159.415032 84.836) (end 158.806 84.226968) (width 0.2) (layer "F.Cu") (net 8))
 (segment (start 157.48 83.82) (end 153.924 83.82) (width 0.2) (layer "F.Cu") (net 7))
 (segment (start 157.988 84.328) (end 157.48 83.82) (width 0.2) (layer "F.Cu") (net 7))
 (segment (start 153.924 83.82) (end 153.924 80.9475) (width 0.2) (layer "F.Cu") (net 7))
 (via (at 157.988 84.328) (size 0.6) (drill 0.3) (layers "F.Cu" "B.Cu") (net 7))
 (segment (start 169.164 92.924) (end 166.345 95.743) (width 0.2) (layer "B.Cu") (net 7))
 (segment (start 155.433 86.883) (end 157.988 84.328) (width 0.2) (layer "B.Cu") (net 7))
 (segment (start 152.307 87.381057) (end 152.805057 86.883) (width 0.2) (layer "B.Cu") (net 7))
 (segment (start 166.345 95.743) (end 153.763372 95.743) (width 0.2) (layer "B.Cu") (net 7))
 (segment (start 153.763372 95.743) (end 152.307 94.286628) (width 0.2) (layer "B.Cu") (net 7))
 (segment (start 152.805057 86.883) (end 155.433 86.883) (width 0.2) (layer "B.Cu") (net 7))
 (segment (start 152.307 94.286628) (end 152.307 87.381057) (width 0.2) (layer "B.Cu") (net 7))
 (segment (start 168.91 91.694) (end 168.817 91.787) (width 0.2) (layer "B.Cu") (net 7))
 (segment (start 170.434 73.406) (end 172.466 71.374) (width 0.2) (layer "F.Cu") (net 2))
 (segment (start 161.285 73.406) (end 170.434 73.406) (width 0.2) (layer "F.Cu") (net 2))
 (segment (start 170.434 77.221) (end 170.434 73.406) (width 0.2) (layer "F.Cu") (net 2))
 (segment (start 172.461 79.248) (end 170.434 77.221) (width 0.2) (layer "F.Cu") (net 2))
 (segment (start 152.414 72.117) (end 152.414 78.5125) (width 0.5) (layer "F.Cu") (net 4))
 (segment (start 152.974 79.0725) (end 152.8295 79.0725) (width 0.2) (layer "F.Cu") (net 4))
 (segment (start 151.7825 80.264) (end 152.974 79.0725) (width 0.5) (layer "F.Cu") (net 4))
 (segment (start 164.841 76.708) (end 163.5635 76.708) (width 0.5) (layer "F.Cu") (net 4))
 (segment (start 152.414 78.5125) (end 152.974 79.0725) (width 0.5) (layer "F.Cu") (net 4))
 (segment (start 163.5635 76.708) (end 161.2115 79.06) (width 0.5) (layer "F.Cu") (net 4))
 (segment (start 160.0355 77.884) (end 154.1625 77.884) (width 0.5) (layer "F.Cu") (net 4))
 (segment (start 161.2115 79.06) (end 160.0355 77.884) (width 0.5) (layer "F.Cu") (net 4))
 (segment (start 154.1625 77.884) (end 152.974 79.0725) (width 0.5) (layer "F.Cu") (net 4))
 (segment (start 153.665 70.866) (end 152.414 72.117) (width 0.5) (layer "F.Cu") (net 4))
 (segment (start 145.288 80.264) (end 151.7825 80.264) (width 0.5) (layer "F.Cu") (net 4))
 (segment (start 156.718 84.582) (end 156.718 85.695) (width 0.2) (layer "F.Cu") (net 14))
 (segment (start 156.718 85.695) (end 159.7535 85.695) (width 0.2) (layer "F.Cu") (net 14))
 (segment (start 154.178 87.884) (end 154.178 90.17) (width 0.2) (layer "F.Cu") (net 14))
 (segment (start 154.874 86.04) (end 154.178 86.736) (width 0.2) (layer "F.Cu") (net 14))
 (segment (start 154.874 85.695) (end 156.718 85.695) (width 0.2) (layer "F.Cu") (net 14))
 (segment (start 154.874 85.695) (end 154.874 86.04) (width 0.2) (layer "F.Cu") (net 14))
 (segment (start 159.7535 85.695) (end 159.8445 85.786) (width 0.2) (layer "F.Cu") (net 14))
 (segment (start 154.178 86.736) (end 154.178 87.884) (width 0.2) (layer "F.Cu") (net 14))
 (via (at 156.718 84.582) (size 0.6) (drill 0.3) (layers "F.Cu" "B.Cu") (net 14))
 (segment (start 154.686 84.582) (end 156.718 84.582) (width 0.2) (layer "B.Cu") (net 14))
 (segment (start 145.288 75.184) (end 154.686 84.582) (width 0.2) (layer "B.Cu") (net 14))
 (segment (start 159.844532 79.0725) (end 160.433032 79.661) (width 0.2) (layer "F.Cu") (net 5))
 (segment (start 152.974 85.695) (end 152.974 87.564) (width 0.2) (layer "F.Cu") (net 5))
 (segment (start 160.433032 79.661) (end 164.428 79.661) (width 0.2) (layer "F.Cu") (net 5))
 (segment (start 152.974 85.695) (end 152.974 80.518032) (width 0.2) (layer "F.Cu") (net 5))
 (segment (start 164.428 79.661) (end 164.841 79.248) (width 0.2) (layer "F.Cu") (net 5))
 (segment (start 154.419532 79.0725) (end 154.874 79.0725) (width 0.2) (layer "F.Cu") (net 5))
 (segment (start 154.874 79.0725) (end 159.844532 79.0725) (width 0.2) (layer "F.Cu") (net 5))
 (segment (start 152.974 80.518032) (end 154.419532 79.0725) (width 0.2) (layer "F.Cu") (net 5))
 (segment (start 152.974 87.564) (end 152.908 87.63) (width 0.2) (layer "F.Cu") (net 5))
 (via (at 152.908 87.63) (size 0.6) (drill 0.3) (layers "F.Cu" "B.Cu") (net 5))
 (segment (start 152.908 87.63) (end 152.908 88.029628) (width 0.2) (layer "B.Cu") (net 5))
 (segment (start 158.257 88.885) (end 159.258 87.884) (width 0.2) (layer "B.Cu") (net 5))
 (segment (start 152.908 88.029628) (end 153.763372 88.885) (width 0.2) (layer "B.Cu") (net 5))
 (segment (start 153.763372 88.885) (end 158.257 88.885) (width 0.2) (layer "B.Cu") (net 5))
 (segment (start 161.986 83.886) (end 159.8445 83.886) (width 0.2) (layer "F.Cu") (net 11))
 (segment (start 161.2115 80.96) (end 159.8445 82.327) (width 0.2) (layer "F.Cu") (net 11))
 (segment (start 159.8445 82.327) (end 159.8445 83.566) (width 0.2) (layer "F.Cu") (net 11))
 (segment (start 162.052 83.82) (end 161.986 83.886) (width 0.2) (layer "F.Cu") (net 11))
 (segment (start 161.2115 80.96) (end 162.626 80.96) (width 0.2) (layer "F.Cu") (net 11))
 (segment (start 162.626 80.96) (end 163.068 80.518) (width 0.2) (layer "F.Cu") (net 11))
 (via (at 163.068 80.518) (size 0.6) (drill 0.3) (layers "F.Cu" "B.Cu") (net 11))
 (via (at 162.052 83.82) (size 0.6) (drill 0.3) (layers "F.Cu" "B.Cu") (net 11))
 (segment (start 162.052 87.376) (end 162.052 83.82) (width 0.2) (layer "B.Cu") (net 11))
 (segment (start 159.258 90.17) (end 162.052 87.376) (width 0.2) (layer "B.Cu") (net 11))
 (segment (start 163.068 80.518) (end 155.956 73.406) (width 0.2) (layer "B.Cu") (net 11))
 (segment (start 155.956 73.406) (end 153.665 73.406) (width 0.2) (layer "B.Cu") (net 11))
 (segment (start 162.814 85.598) (end 162.814 88.9) (width 0.2) (layer "F.Cu") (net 1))
 (segment (start 162.814 88.9) (end 159.258 92.456) (width 0.2) (layer "F.Cu") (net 1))
 (via (at 162.814 85.598) (size 0.6) (drill 0.3) (layers "F.Cu" "B.Cu") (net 1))
 (segment (start 172.461 81.788) (end 166.624 81.788) (width 0.2) (layer "B.Cu") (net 1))
 (segment (start 166.624 81.788) (end 162.814 85.598) (width 0.2) (layer "B.Cu") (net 1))
 (segment (start 159.258 94.742) (end 158.257 93.741) (width 0.2) (layer "B.Cu") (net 9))
 (segment (start 163.669 80.766943) (end 163.669 78.33) (width 0.2) (layer "B.Cu") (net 9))
 (segment (start 158.257 89.755372) (end 158.843372 89.169) (width 0.2) (layer "B.Cu") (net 9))
 (segment (start 158.257 93.741) (end 158.257 89.755372) (width 0.2) (layer "B.Cu") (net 9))
 (segment (start 163.669 78.33) (end 161.285 75.946) (width 0.2) (layer "B.Cu") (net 9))
 (segment (start 161.451 87.390628) (end 161.451 82.984943) (width 0.2) (layer "B.Cu") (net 9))
 (segment (start 161.451 82.984943) (end 163.669 80.766943) (width 0.2) (layer "B.Cu") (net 9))
 (segment (start 159.672628 89.169) (end 161.451 87.390628) (width 0.2) (layer "B.Cu") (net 9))
 (segment (start 158.843372 89.169) (end 159.672628 89.169) (width 0.2) (layer "B.Cu") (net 9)))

